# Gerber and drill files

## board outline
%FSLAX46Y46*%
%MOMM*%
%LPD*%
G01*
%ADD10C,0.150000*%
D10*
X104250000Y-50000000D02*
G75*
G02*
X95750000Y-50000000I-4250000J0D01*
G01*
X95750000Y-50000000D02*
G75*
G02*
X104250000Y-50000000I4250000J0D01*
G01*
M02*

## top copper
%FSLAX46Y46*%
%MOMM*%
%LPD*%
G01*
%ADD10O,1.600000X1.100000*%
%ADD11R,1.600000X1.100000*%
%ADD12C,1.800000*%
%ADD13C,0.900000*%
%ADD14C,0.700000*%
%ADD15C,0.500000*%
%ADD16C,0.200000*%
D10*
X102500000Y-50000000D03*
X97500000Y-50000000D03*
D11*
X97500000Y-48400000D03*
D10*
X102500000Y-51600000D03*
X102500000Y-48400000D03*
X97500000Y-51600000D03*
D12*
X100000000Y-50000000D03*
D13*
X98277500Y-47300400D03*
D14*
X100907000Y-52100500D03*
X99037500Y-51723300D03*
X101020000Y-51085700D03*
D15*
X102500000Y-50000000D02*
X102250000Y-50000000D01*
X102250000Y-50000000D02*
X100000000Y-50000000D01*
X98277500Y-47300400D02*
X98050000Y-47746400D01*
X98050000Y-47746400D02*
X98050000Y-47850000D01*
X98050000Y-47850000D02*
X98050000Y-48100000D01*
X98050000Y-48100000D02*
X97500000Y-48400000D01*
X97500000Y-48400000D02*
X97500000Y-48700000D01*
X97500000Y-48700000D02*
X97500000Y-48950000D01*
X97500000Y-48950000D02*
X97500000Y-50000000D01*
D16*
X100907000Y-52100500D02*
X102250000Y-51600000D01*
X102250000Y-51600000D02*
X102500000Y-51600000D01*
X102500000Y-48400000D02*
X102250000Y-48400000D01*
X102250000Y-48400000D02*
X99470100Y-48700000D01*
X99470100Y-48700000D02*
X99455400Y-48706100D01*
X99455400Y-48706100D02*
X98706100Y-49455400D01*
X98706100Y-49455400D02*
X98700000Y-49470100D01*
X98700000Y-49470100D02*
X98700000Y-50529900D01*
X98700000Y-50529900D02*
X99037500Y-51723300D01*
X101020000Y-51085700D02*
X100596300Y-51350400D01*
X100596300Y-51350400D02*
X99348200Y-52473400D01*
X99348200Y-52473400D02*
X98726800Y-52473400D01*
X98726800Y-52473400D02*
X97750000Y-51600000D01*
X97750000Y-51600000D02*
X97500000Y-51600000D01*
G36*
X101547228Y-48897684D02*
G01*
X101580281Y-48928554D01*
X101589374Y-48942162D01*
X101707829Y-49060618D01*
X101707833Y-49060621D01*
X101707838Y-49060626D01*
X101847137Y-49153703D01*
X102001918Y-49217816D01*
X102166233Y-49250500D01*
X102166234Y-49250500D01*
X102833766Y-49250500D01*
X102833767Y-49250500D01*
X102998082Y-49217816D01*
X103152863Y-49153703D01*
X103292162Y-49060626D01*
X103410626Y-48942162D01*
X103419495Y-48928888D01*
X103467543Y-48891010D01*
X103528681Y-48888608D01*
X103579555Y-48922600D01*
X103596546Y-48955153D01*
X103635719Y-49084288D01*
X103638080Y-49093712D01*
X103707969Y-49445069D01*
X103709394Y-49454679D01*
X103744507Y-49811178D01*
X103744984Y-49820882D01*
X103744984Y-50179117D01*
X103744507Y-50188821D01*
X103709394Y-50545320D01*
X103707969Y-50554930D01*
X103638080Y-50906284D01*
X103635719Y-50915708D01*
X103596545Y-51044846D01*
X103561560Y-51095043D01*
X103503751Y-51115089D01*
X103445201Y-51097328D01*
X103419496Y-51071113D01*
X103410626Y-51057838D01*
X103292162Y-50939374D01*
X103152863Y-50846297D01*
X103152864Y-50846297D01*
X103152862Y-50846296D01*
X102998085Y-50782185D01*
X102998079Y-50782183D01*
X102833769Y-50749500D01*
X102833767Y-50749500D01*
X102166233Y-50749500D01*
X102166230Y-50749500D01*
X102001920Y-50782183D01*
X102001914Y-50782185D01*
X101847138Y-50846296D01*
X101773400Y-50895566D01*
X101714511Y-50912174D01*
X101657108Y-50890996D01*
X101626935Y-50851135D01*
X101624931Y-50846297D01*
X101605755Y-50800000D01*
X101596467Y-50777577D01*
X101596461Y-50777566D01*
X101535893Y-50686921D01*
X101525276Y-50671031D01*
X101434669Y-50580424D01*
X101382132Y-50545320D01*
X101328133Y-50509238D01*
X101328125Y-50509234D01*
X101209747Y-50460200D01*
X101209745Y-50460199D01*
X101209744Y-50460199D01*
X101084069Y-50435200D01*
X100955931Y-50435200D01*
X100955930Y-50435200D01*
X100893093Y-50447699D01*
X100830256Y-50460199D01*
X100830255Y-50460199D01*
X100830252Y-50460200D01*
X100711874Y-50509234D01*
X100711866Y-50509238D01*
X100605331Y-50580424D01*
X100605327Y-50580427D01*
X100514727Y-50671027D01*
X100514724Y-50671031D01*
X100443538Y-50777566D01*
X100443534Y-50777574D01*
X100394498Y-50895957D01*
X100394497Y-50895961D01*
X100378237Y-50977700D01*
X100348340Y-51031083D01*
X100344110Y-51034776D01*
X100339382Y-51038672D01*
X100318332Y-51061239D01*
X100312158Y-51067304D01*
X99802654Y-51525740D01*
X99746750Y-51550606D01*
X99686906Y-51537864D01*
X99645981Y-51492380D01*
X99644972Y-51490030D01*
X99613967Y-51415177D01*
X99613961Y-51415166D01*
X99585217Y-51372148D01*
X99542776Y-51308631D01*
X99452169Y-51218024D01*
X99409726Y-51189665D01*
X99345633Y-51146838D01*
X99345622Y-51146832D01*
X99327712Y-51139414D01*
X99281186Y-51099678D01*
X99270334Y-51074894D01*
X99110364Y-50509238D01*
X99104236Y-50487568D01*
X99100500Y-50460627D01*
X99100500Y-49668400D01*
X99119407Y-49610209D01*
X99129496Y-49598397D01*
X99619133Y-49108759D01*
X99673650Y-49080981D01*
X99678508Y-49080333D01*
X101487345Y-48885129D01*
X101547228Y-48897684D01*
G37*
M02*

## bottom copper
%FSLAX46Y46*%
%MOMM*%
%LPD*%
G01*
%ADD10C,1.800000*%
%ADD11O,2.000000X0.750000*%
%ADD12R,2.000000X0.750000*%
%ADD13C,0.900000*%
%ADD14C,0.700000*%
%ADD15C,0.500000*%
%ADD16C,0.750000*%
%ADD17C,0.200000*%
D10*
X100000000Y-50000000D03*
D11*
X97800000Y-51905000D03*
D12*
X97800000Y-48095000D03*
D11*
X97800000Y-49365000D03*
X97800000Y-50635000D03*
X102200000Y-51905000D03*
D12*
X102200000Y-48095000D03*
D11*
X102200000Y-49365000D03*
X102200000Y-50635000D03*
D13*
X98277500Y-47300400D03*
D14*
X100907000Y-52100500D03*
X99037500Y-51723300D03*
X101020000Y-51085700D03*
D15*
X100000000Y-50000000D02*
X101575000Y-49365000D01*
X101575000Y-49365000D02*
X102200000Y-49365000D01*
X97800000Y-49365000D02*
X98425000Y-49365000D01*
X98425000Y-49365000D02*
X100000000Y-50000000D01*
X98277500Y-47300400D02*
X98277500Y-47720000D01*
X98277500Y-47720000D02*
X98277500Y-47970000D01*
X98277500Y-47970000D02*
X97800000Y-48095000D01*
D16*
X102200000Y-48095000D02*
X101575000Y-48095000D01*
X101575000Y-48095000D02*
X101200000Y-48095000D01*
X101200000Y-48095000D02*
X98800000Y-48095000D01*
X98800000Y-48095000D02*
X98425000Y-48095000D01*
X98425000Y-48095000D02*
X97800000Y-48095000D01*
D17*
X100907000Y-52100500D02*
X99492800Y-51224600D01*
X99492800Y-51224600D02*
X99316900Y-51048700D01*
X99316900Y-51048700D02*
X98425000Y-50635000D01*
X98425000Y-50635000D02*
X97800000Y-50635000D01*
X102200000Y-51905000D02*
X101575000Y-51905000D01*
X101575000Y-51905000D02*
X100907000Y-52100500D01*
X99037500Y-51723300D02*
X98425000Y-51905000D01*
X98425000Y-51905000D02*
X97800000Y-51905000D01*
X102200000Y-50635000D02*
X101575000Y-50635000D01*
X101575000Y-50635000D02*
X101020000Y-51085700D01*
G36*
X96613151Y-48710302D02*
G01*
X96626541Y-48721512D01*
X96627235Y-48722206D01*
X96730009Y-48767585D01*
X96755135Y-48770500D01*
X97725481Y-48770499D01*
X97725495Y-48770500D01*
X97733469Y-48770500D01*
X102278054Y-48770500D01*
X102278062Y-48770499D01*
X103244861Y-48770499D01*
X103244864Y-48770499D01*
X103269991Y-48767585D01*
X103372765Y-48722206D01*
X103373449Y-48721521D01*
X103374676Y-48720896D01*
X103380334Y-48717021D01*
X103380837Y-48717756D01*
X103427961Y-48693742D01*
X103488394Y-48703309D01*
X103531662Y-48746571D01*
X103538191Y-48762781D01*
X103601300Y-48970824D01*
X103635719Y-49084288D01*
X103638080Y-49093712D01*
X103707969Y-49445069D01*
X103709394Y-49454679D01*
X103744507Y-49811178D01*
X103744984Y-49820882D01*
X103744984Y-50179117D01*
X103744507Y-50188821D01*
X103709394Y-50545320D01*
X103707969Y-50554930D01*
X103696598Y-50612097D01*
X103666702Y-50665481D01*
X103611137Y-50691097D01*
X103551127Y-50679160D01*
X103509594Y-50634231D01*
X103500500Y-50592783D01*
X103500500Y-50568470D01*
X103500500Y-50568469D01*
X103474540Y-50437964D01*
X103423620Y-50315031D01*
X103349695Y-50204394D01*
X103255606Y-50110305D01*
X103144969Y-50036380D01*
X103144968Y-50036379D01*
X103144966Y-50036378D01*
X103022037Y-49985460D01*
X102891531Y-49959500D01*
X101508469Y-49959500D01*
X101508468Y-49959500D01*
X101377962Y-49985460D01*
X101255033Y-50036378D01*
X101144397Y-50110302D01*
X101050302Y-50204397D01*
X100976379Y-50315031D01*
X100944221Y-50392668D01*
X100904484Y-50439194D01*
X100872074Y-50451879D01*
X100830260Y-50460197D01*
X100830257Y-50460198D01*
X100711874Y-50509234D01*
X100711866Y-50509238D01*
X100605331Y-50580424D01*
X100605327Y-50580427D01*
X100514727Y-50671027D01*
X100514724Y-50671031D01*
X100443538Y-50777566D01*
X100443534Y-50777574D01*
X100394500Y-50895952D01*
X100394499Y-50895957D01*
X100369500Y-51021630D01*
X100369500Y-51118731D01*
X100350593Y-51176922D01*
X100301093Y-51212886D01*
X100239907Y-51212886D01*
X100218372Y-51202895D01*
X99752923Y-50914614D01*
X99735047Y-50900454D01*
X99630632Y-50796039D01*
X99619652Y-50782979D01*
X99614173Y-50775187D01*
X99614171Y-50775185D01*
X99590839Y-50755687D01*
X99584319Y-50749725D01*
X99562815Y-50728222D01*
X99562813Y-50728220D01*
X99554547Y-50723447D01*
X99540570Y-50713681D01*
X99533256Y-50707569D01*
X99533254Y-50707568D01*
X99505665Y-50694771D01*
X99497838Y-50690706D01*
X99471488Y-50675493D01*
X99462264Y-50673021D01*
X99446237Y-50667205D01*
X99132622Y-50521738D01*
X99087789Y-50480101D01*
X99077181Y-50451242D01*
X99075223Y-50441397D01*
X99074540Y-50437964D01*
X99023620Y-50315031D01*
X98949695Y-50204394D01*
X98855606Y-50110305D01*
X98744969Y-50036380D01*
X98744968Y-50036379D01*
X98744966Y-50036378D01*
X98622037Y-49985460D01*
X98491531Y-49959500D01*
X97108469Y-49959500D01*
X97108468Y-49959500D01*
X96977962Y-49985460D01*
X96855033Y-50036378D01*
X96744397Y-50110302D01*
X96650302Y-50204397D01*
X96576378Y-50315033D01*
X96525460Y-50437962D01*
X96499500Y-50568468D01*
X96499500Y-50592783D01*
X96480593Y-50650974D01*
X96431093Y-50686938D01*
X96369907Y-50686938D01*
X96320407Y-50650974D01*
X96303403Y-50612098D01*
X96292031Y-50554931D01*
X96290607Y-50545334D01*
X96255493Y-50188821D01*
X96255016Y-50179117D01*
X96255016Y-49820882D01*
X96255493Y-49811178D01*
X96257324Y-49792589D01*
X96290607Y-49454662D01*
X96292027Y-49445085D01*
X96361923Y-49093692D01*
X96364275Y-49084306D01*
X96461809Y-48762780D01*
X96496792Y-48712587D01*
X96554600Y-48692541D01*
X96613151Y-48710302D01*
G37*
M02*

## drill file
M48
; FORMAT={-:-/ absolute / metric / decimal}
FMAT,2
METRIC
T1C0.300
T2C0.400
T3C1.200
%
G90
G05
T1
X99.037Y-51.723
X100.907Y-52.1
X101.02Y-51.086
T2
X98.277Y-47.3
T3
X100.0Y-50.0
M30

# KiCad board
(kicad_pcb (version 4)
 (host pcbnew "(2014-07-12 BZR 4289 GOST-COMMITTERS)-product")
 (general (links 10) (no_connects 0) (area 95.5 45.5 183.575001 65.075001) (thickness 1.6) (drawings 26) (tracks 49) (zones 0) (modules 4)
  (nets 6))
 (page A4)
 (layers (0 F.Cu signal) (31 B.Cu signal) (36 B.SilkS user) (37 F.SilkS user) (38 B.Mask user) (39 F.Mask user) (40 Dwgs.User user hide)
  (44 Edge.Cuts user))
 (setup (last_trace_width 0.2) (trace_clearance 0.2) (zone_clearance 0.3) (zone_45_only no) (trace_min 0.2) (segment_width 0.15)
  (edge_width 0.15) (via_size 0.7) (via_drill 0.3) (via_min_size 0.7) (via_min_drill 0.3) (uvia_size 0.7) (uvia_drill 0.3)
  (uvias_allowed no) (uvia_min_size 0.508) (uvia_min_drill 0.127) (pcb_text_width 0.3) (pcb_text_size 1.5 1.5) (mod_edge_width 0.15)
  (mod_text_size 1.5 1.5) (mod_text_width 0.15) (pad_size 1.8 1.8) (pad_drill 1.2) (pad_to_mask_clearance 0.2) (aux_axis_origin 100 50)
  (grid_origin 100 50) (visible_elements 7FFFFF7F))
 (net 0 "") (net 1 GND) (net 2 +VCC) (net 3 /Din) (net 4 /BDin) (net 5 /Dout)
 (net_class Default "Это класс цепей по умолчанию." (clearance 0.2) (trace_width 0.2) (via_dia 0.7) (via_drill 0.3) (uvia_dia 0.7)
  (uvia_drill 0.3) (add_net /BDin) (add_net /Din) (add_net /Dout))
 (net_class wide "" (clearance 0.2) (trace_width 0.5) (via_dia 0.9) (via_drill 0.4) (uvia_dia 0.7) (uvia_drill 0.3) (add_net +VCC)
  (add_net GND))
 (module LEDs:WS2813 (layer F.Cu) (at 100 50 180)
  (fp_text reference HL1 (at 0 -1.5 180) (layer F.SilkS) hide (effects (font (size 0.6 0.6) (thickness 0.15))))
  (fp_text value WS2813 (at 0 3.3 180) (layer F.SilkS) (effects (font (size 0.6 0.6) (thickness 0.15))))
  (pad 5 smd oval (at -2.5 0 180) (size 1.6 1.1) (layers F.Cu F.Mask) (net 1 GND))
  (pad 2 smd oval (at 2.5 0 180) (size 1.6 1.1) (layers F.Cu F.Mask) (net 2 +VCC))
  (pad 1 smd rect (at 2.5 1.6 180) (size 1.6 1.1) (layers F.Cu F.Mask) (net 2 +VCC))
  (pad 4 smd oval (at -2.5 -1.6 180) (size 1.6 1.1) (layers F.Cu F.Mask) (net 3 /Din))
  (pad 6 smd oval (at -2.5 1.6 180) (size 1.6 1.1) (layers F.Cu F.Mask) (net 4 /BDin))
  (pad 3 smd oval (at 2.5 -1.6 180) (size 1.6 1.1) (layers F.Cu F.Mask) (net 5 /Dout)))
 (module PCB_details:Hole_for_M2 (layer F.Cu) (at 100 50 270)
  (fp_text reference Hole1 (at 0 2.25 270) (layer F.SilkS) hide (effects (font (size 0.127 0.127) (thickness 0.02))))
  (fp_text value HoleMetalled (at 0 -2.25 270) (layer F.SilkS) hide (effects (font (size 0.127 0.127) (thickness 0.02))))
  (pad H thru_hole circle (at 0 0 270) (size 1.8 1.8) (drill 1.2) (layers *.Cu *.Mask) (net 1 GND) (zone_connect 2)))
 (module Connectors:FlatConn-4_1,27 (layer B.Cu) (at 97.8 50 270)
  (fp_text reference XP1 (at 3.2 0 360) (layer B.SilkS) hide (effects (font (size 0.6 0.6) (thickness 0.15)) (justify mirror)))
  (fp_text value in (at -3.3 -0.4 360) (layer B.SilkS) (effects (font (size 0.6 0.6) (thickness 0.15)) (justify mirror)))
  (pad 4 smd oval (at 1.905 0 270) (size 0.75 2) (layers B.Cu B.Mask) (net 4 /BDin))
  (pad 1 smd rect (at -1.905 0 270) (size 0.75 2) (layers B.Cu B.Mask) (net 2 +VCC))
  (pad 2 smd oval (at -0.635 0 270) (size 0.75 2) (layers B.Cu B.Mask) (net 1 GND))
  (pad 3 smd oval (at 0.635 0 270) (size 0.75 2) (layers B.Cu B.Mask) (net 3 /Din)))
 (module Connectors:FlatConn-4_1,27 (layer B.Cu) (at 102.2 50 270)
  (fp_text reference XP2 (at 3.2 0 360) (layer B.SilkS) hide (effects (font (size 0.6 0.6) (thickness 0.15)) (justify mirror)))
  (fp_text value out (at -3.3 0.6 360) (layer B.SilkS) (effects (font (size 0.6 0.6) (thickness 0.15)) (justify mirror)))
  (pad 4 smd oval (at 1.905 0 270) (size 0.75 2) (layers B.Cu B.Mask) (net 3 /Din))
  (pad 1 smd rect (at -1.905 0 270) (size 0.75 2) (layers B.Cu B.Mask) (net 2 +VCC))
  (pad 2 smd oval (at -0.635 0 270) (size 0.75 2) (layers B.Cu B.Mask) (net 1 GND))
  (pad 3 smd oval (at 0.635 0 270) (size 0.75 2) (layers B.Cu B.Mask) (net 5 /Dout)))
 (gr_circle (center 100 50) (end 95.75 50) (layer Edge.Cuts) (width 0.15))
 (segment (start 102.5 50) (end 102.25 50) (width 0.5) (layer F.Cu) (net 1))
 (segment (start 102.25 50) (end 100 50) (width 0.5) (layer F.Cu) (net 1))
 (segment (start 100 50) (end 101.575 49.365) (width 0.5) (layer B.Cu) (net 1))
 (segment (start 101.575 49.365) (end 102.2 49.365) (width 0.5) (layer B.Cu) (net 1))
 (segment (start 97.8 49.365) (end 98.425 49.365) (width 0.5) (layer B.Cu) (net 1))
 (segment (start 98.425 49.365) (end 100 50) (width 0.5) (layer B.Cu) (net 1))
 (segment (start 98.2775 47.3004) (end 98.05 47.7464) (width 0.5) (layer F.Cu) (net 2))
 (segment (start 98.05 47.7464) (end 98.05 47.85) (width 0.5) (layer F.Cu) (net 2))
 (segment (start 98.05 47.85) (end 98.05 48.1) (width 0.5) (layer F.Cu) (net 2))
 (segment (start 98.05 48.1) (end 97.5 48.4) (width 0.5) (layer F.Cu) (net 2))
 (segment (start 97.5 48.4) (end 97.5 48.7) (width 0.5) (layer F.Cu) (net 2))
 (segment (start 97.5 48.7) (end 97.5 48.95) (width 0.5) (layer F.Cu) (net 2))
 (segment (start 97.5 48.95) (end 97.5 50) (width 0.5) (layer F.Cu) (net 2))
 (segment (start 98.2775 47.3004) (end 98.2775 47.72) (width 0.5) (layer B.Cu) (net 2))
 (segment (start 98.2775 47.72) (end 98.2775 47.97) (width 0.5) (layer B.Cu) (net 2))
 (segment (start 98.2775 47.97) (end 97.8 48.095) (width 0.5) (layer B.Cu) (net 2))
 (segment (start 102.2 48.095) (end 101.575 48.095) (width 0.75) (layer B.Cu) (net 2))
 (segment (start 101.575 48.095) (end 101.2 48.095) (width 0.75) (layer B.Cu) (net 2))
 (segment (start 101.2 48.095) (end 98.8 48.095) (width 0.75) (layer B.Cu) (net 2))
 (segment (start 98.8 48.095) (end 98.425 48.095) (width 0.75) (layer B.Cu) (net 2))
 (segment (start 98.425 48.095) (end 97.8 48.095) (width 0.75) (layer B.Cu) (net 2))
 (via (at 98.2775 47.3004) (size 0.9) (layers F.Cu B.Cu) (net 2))
 (segment (start 100.907 52.1005) (end 102.25 51.6) (width 0.2) (layer F.Cu) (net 3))
 (segment (start 102.25 51.6) (end 102.5 51.6) (width 0.2) (layer F.Cu) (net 3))
 (segment (start 100.907 52.1005) (end 99.4928 51.2246) (width 0.2) (layer B.Cu) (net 3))
 (segment (start 99.4928 51.2246) (end 99.3169 51.0487) (width 0.2) (layer B.Cu) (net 3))
 (segment (start 99.3169 51.0487) (end 98.425 50.635) (width 0.2) (layer B.Cu) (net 3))
 (segment (start 98.425 50.635) (end 97.8 50.635) (width 0.2) (layer B.Cu) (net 3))
 (segment (start 102.2 51.905) (end 101.575 51.905) (width 0.2) (layer B.Cu) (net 3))
 (segment (start 101.575 51.905) (end 100.907 52.1005) (width 0.2) (layer B.Cu) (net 3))
 (via (at 100.907 52.1005) (size 0.7) (layers F.Cu B.Cu) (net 3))
 (segment (start 102.5 48.4) (end 102.25 48.4) (width 0.2) (layer F.Cu) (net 4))
 (segment (start 102.25 48.4) (end 99.4701 48.7) (width 0.2) (layer F.Cu) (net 4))
 (segment (start 99.4701 48.7) (end 99.4554 48.7061) (width 0.2) (layer F.Cu) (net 4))
 (segment (start 99.4554 48.7061) (end 98.7061 49.4554) (width 0.2) (layer F.Cu) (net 4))
 (segment (start 98.7061 49.4554) (end 98.7 49.4701) (width 0.2) (layer F.Cu) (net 4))
 (segment (start 98.7 49.4701) (end 98.7 50.5299) (width 0.2) (layer F.Cu) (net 4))
 (segment (start 98.7 50.5299) (end 99.0375 51.7233) (width 0.2) (layer F.Cu) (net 4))
 (segment (start 99.0375 51.7233) (end 98.425 51.905) (width 0.2) (layer B.Cu) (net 4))
 (segment (start 98.425 51.905) (end 97.8 51.905) (width 0.2) (layer B.Cu) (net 4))
 (via (at 99.0375 51.7233) (size 0.7) (layers F.Cu B.Cu) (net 4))
 (segment (start 101.02 51.0857) (end 100.5963 51.3504) (width 0.2) (layer F.Cu) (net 5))
 (segment (start 100.5963 51.3504) (end 99.3482 52.4734) (width 0.2) (layer F.Cu) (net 5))
 (segment (start 99.3482 52.4734) (end 98.7268 52.4734) (width 0.2) (layer F.Cu) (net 5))
 (segment (start 98.7268 52.4734) (end 97.75 51.6) (width 0.2) (layer F.Cu) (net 5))
 (segment (start 97.75 51.6) (end 97.5 51.6) (width 0.2) (layer F.Cu) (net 5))
 (segment (start 102.2 50.635) (end 101.575 50.635) (width 0.2) (layer B.Cu) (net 5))
 (segment (start 101.575 50.635) (end 101.02 51.0857) (width 0.2) (layer B.Cu) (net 5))
 (via (at 101.02 51.0857) (size 0.7) (layers F.Cu B.Cu) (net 5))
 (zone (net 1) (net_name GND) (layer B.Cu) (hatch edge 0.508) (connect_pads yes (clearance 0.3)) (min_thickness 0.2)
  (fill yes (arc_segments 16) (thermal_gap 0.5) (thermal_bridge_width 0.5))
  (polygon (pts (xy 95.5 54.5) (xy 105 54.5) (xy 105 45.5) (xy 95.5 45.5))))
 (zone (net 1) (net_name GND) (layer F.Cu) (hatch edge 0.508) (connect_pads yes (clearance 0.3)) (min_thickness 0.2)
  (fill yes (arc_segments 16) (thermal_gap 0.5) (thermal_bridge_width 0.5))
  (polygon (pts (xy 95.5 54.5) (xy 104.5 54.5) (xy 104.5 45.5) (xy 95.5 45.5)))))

